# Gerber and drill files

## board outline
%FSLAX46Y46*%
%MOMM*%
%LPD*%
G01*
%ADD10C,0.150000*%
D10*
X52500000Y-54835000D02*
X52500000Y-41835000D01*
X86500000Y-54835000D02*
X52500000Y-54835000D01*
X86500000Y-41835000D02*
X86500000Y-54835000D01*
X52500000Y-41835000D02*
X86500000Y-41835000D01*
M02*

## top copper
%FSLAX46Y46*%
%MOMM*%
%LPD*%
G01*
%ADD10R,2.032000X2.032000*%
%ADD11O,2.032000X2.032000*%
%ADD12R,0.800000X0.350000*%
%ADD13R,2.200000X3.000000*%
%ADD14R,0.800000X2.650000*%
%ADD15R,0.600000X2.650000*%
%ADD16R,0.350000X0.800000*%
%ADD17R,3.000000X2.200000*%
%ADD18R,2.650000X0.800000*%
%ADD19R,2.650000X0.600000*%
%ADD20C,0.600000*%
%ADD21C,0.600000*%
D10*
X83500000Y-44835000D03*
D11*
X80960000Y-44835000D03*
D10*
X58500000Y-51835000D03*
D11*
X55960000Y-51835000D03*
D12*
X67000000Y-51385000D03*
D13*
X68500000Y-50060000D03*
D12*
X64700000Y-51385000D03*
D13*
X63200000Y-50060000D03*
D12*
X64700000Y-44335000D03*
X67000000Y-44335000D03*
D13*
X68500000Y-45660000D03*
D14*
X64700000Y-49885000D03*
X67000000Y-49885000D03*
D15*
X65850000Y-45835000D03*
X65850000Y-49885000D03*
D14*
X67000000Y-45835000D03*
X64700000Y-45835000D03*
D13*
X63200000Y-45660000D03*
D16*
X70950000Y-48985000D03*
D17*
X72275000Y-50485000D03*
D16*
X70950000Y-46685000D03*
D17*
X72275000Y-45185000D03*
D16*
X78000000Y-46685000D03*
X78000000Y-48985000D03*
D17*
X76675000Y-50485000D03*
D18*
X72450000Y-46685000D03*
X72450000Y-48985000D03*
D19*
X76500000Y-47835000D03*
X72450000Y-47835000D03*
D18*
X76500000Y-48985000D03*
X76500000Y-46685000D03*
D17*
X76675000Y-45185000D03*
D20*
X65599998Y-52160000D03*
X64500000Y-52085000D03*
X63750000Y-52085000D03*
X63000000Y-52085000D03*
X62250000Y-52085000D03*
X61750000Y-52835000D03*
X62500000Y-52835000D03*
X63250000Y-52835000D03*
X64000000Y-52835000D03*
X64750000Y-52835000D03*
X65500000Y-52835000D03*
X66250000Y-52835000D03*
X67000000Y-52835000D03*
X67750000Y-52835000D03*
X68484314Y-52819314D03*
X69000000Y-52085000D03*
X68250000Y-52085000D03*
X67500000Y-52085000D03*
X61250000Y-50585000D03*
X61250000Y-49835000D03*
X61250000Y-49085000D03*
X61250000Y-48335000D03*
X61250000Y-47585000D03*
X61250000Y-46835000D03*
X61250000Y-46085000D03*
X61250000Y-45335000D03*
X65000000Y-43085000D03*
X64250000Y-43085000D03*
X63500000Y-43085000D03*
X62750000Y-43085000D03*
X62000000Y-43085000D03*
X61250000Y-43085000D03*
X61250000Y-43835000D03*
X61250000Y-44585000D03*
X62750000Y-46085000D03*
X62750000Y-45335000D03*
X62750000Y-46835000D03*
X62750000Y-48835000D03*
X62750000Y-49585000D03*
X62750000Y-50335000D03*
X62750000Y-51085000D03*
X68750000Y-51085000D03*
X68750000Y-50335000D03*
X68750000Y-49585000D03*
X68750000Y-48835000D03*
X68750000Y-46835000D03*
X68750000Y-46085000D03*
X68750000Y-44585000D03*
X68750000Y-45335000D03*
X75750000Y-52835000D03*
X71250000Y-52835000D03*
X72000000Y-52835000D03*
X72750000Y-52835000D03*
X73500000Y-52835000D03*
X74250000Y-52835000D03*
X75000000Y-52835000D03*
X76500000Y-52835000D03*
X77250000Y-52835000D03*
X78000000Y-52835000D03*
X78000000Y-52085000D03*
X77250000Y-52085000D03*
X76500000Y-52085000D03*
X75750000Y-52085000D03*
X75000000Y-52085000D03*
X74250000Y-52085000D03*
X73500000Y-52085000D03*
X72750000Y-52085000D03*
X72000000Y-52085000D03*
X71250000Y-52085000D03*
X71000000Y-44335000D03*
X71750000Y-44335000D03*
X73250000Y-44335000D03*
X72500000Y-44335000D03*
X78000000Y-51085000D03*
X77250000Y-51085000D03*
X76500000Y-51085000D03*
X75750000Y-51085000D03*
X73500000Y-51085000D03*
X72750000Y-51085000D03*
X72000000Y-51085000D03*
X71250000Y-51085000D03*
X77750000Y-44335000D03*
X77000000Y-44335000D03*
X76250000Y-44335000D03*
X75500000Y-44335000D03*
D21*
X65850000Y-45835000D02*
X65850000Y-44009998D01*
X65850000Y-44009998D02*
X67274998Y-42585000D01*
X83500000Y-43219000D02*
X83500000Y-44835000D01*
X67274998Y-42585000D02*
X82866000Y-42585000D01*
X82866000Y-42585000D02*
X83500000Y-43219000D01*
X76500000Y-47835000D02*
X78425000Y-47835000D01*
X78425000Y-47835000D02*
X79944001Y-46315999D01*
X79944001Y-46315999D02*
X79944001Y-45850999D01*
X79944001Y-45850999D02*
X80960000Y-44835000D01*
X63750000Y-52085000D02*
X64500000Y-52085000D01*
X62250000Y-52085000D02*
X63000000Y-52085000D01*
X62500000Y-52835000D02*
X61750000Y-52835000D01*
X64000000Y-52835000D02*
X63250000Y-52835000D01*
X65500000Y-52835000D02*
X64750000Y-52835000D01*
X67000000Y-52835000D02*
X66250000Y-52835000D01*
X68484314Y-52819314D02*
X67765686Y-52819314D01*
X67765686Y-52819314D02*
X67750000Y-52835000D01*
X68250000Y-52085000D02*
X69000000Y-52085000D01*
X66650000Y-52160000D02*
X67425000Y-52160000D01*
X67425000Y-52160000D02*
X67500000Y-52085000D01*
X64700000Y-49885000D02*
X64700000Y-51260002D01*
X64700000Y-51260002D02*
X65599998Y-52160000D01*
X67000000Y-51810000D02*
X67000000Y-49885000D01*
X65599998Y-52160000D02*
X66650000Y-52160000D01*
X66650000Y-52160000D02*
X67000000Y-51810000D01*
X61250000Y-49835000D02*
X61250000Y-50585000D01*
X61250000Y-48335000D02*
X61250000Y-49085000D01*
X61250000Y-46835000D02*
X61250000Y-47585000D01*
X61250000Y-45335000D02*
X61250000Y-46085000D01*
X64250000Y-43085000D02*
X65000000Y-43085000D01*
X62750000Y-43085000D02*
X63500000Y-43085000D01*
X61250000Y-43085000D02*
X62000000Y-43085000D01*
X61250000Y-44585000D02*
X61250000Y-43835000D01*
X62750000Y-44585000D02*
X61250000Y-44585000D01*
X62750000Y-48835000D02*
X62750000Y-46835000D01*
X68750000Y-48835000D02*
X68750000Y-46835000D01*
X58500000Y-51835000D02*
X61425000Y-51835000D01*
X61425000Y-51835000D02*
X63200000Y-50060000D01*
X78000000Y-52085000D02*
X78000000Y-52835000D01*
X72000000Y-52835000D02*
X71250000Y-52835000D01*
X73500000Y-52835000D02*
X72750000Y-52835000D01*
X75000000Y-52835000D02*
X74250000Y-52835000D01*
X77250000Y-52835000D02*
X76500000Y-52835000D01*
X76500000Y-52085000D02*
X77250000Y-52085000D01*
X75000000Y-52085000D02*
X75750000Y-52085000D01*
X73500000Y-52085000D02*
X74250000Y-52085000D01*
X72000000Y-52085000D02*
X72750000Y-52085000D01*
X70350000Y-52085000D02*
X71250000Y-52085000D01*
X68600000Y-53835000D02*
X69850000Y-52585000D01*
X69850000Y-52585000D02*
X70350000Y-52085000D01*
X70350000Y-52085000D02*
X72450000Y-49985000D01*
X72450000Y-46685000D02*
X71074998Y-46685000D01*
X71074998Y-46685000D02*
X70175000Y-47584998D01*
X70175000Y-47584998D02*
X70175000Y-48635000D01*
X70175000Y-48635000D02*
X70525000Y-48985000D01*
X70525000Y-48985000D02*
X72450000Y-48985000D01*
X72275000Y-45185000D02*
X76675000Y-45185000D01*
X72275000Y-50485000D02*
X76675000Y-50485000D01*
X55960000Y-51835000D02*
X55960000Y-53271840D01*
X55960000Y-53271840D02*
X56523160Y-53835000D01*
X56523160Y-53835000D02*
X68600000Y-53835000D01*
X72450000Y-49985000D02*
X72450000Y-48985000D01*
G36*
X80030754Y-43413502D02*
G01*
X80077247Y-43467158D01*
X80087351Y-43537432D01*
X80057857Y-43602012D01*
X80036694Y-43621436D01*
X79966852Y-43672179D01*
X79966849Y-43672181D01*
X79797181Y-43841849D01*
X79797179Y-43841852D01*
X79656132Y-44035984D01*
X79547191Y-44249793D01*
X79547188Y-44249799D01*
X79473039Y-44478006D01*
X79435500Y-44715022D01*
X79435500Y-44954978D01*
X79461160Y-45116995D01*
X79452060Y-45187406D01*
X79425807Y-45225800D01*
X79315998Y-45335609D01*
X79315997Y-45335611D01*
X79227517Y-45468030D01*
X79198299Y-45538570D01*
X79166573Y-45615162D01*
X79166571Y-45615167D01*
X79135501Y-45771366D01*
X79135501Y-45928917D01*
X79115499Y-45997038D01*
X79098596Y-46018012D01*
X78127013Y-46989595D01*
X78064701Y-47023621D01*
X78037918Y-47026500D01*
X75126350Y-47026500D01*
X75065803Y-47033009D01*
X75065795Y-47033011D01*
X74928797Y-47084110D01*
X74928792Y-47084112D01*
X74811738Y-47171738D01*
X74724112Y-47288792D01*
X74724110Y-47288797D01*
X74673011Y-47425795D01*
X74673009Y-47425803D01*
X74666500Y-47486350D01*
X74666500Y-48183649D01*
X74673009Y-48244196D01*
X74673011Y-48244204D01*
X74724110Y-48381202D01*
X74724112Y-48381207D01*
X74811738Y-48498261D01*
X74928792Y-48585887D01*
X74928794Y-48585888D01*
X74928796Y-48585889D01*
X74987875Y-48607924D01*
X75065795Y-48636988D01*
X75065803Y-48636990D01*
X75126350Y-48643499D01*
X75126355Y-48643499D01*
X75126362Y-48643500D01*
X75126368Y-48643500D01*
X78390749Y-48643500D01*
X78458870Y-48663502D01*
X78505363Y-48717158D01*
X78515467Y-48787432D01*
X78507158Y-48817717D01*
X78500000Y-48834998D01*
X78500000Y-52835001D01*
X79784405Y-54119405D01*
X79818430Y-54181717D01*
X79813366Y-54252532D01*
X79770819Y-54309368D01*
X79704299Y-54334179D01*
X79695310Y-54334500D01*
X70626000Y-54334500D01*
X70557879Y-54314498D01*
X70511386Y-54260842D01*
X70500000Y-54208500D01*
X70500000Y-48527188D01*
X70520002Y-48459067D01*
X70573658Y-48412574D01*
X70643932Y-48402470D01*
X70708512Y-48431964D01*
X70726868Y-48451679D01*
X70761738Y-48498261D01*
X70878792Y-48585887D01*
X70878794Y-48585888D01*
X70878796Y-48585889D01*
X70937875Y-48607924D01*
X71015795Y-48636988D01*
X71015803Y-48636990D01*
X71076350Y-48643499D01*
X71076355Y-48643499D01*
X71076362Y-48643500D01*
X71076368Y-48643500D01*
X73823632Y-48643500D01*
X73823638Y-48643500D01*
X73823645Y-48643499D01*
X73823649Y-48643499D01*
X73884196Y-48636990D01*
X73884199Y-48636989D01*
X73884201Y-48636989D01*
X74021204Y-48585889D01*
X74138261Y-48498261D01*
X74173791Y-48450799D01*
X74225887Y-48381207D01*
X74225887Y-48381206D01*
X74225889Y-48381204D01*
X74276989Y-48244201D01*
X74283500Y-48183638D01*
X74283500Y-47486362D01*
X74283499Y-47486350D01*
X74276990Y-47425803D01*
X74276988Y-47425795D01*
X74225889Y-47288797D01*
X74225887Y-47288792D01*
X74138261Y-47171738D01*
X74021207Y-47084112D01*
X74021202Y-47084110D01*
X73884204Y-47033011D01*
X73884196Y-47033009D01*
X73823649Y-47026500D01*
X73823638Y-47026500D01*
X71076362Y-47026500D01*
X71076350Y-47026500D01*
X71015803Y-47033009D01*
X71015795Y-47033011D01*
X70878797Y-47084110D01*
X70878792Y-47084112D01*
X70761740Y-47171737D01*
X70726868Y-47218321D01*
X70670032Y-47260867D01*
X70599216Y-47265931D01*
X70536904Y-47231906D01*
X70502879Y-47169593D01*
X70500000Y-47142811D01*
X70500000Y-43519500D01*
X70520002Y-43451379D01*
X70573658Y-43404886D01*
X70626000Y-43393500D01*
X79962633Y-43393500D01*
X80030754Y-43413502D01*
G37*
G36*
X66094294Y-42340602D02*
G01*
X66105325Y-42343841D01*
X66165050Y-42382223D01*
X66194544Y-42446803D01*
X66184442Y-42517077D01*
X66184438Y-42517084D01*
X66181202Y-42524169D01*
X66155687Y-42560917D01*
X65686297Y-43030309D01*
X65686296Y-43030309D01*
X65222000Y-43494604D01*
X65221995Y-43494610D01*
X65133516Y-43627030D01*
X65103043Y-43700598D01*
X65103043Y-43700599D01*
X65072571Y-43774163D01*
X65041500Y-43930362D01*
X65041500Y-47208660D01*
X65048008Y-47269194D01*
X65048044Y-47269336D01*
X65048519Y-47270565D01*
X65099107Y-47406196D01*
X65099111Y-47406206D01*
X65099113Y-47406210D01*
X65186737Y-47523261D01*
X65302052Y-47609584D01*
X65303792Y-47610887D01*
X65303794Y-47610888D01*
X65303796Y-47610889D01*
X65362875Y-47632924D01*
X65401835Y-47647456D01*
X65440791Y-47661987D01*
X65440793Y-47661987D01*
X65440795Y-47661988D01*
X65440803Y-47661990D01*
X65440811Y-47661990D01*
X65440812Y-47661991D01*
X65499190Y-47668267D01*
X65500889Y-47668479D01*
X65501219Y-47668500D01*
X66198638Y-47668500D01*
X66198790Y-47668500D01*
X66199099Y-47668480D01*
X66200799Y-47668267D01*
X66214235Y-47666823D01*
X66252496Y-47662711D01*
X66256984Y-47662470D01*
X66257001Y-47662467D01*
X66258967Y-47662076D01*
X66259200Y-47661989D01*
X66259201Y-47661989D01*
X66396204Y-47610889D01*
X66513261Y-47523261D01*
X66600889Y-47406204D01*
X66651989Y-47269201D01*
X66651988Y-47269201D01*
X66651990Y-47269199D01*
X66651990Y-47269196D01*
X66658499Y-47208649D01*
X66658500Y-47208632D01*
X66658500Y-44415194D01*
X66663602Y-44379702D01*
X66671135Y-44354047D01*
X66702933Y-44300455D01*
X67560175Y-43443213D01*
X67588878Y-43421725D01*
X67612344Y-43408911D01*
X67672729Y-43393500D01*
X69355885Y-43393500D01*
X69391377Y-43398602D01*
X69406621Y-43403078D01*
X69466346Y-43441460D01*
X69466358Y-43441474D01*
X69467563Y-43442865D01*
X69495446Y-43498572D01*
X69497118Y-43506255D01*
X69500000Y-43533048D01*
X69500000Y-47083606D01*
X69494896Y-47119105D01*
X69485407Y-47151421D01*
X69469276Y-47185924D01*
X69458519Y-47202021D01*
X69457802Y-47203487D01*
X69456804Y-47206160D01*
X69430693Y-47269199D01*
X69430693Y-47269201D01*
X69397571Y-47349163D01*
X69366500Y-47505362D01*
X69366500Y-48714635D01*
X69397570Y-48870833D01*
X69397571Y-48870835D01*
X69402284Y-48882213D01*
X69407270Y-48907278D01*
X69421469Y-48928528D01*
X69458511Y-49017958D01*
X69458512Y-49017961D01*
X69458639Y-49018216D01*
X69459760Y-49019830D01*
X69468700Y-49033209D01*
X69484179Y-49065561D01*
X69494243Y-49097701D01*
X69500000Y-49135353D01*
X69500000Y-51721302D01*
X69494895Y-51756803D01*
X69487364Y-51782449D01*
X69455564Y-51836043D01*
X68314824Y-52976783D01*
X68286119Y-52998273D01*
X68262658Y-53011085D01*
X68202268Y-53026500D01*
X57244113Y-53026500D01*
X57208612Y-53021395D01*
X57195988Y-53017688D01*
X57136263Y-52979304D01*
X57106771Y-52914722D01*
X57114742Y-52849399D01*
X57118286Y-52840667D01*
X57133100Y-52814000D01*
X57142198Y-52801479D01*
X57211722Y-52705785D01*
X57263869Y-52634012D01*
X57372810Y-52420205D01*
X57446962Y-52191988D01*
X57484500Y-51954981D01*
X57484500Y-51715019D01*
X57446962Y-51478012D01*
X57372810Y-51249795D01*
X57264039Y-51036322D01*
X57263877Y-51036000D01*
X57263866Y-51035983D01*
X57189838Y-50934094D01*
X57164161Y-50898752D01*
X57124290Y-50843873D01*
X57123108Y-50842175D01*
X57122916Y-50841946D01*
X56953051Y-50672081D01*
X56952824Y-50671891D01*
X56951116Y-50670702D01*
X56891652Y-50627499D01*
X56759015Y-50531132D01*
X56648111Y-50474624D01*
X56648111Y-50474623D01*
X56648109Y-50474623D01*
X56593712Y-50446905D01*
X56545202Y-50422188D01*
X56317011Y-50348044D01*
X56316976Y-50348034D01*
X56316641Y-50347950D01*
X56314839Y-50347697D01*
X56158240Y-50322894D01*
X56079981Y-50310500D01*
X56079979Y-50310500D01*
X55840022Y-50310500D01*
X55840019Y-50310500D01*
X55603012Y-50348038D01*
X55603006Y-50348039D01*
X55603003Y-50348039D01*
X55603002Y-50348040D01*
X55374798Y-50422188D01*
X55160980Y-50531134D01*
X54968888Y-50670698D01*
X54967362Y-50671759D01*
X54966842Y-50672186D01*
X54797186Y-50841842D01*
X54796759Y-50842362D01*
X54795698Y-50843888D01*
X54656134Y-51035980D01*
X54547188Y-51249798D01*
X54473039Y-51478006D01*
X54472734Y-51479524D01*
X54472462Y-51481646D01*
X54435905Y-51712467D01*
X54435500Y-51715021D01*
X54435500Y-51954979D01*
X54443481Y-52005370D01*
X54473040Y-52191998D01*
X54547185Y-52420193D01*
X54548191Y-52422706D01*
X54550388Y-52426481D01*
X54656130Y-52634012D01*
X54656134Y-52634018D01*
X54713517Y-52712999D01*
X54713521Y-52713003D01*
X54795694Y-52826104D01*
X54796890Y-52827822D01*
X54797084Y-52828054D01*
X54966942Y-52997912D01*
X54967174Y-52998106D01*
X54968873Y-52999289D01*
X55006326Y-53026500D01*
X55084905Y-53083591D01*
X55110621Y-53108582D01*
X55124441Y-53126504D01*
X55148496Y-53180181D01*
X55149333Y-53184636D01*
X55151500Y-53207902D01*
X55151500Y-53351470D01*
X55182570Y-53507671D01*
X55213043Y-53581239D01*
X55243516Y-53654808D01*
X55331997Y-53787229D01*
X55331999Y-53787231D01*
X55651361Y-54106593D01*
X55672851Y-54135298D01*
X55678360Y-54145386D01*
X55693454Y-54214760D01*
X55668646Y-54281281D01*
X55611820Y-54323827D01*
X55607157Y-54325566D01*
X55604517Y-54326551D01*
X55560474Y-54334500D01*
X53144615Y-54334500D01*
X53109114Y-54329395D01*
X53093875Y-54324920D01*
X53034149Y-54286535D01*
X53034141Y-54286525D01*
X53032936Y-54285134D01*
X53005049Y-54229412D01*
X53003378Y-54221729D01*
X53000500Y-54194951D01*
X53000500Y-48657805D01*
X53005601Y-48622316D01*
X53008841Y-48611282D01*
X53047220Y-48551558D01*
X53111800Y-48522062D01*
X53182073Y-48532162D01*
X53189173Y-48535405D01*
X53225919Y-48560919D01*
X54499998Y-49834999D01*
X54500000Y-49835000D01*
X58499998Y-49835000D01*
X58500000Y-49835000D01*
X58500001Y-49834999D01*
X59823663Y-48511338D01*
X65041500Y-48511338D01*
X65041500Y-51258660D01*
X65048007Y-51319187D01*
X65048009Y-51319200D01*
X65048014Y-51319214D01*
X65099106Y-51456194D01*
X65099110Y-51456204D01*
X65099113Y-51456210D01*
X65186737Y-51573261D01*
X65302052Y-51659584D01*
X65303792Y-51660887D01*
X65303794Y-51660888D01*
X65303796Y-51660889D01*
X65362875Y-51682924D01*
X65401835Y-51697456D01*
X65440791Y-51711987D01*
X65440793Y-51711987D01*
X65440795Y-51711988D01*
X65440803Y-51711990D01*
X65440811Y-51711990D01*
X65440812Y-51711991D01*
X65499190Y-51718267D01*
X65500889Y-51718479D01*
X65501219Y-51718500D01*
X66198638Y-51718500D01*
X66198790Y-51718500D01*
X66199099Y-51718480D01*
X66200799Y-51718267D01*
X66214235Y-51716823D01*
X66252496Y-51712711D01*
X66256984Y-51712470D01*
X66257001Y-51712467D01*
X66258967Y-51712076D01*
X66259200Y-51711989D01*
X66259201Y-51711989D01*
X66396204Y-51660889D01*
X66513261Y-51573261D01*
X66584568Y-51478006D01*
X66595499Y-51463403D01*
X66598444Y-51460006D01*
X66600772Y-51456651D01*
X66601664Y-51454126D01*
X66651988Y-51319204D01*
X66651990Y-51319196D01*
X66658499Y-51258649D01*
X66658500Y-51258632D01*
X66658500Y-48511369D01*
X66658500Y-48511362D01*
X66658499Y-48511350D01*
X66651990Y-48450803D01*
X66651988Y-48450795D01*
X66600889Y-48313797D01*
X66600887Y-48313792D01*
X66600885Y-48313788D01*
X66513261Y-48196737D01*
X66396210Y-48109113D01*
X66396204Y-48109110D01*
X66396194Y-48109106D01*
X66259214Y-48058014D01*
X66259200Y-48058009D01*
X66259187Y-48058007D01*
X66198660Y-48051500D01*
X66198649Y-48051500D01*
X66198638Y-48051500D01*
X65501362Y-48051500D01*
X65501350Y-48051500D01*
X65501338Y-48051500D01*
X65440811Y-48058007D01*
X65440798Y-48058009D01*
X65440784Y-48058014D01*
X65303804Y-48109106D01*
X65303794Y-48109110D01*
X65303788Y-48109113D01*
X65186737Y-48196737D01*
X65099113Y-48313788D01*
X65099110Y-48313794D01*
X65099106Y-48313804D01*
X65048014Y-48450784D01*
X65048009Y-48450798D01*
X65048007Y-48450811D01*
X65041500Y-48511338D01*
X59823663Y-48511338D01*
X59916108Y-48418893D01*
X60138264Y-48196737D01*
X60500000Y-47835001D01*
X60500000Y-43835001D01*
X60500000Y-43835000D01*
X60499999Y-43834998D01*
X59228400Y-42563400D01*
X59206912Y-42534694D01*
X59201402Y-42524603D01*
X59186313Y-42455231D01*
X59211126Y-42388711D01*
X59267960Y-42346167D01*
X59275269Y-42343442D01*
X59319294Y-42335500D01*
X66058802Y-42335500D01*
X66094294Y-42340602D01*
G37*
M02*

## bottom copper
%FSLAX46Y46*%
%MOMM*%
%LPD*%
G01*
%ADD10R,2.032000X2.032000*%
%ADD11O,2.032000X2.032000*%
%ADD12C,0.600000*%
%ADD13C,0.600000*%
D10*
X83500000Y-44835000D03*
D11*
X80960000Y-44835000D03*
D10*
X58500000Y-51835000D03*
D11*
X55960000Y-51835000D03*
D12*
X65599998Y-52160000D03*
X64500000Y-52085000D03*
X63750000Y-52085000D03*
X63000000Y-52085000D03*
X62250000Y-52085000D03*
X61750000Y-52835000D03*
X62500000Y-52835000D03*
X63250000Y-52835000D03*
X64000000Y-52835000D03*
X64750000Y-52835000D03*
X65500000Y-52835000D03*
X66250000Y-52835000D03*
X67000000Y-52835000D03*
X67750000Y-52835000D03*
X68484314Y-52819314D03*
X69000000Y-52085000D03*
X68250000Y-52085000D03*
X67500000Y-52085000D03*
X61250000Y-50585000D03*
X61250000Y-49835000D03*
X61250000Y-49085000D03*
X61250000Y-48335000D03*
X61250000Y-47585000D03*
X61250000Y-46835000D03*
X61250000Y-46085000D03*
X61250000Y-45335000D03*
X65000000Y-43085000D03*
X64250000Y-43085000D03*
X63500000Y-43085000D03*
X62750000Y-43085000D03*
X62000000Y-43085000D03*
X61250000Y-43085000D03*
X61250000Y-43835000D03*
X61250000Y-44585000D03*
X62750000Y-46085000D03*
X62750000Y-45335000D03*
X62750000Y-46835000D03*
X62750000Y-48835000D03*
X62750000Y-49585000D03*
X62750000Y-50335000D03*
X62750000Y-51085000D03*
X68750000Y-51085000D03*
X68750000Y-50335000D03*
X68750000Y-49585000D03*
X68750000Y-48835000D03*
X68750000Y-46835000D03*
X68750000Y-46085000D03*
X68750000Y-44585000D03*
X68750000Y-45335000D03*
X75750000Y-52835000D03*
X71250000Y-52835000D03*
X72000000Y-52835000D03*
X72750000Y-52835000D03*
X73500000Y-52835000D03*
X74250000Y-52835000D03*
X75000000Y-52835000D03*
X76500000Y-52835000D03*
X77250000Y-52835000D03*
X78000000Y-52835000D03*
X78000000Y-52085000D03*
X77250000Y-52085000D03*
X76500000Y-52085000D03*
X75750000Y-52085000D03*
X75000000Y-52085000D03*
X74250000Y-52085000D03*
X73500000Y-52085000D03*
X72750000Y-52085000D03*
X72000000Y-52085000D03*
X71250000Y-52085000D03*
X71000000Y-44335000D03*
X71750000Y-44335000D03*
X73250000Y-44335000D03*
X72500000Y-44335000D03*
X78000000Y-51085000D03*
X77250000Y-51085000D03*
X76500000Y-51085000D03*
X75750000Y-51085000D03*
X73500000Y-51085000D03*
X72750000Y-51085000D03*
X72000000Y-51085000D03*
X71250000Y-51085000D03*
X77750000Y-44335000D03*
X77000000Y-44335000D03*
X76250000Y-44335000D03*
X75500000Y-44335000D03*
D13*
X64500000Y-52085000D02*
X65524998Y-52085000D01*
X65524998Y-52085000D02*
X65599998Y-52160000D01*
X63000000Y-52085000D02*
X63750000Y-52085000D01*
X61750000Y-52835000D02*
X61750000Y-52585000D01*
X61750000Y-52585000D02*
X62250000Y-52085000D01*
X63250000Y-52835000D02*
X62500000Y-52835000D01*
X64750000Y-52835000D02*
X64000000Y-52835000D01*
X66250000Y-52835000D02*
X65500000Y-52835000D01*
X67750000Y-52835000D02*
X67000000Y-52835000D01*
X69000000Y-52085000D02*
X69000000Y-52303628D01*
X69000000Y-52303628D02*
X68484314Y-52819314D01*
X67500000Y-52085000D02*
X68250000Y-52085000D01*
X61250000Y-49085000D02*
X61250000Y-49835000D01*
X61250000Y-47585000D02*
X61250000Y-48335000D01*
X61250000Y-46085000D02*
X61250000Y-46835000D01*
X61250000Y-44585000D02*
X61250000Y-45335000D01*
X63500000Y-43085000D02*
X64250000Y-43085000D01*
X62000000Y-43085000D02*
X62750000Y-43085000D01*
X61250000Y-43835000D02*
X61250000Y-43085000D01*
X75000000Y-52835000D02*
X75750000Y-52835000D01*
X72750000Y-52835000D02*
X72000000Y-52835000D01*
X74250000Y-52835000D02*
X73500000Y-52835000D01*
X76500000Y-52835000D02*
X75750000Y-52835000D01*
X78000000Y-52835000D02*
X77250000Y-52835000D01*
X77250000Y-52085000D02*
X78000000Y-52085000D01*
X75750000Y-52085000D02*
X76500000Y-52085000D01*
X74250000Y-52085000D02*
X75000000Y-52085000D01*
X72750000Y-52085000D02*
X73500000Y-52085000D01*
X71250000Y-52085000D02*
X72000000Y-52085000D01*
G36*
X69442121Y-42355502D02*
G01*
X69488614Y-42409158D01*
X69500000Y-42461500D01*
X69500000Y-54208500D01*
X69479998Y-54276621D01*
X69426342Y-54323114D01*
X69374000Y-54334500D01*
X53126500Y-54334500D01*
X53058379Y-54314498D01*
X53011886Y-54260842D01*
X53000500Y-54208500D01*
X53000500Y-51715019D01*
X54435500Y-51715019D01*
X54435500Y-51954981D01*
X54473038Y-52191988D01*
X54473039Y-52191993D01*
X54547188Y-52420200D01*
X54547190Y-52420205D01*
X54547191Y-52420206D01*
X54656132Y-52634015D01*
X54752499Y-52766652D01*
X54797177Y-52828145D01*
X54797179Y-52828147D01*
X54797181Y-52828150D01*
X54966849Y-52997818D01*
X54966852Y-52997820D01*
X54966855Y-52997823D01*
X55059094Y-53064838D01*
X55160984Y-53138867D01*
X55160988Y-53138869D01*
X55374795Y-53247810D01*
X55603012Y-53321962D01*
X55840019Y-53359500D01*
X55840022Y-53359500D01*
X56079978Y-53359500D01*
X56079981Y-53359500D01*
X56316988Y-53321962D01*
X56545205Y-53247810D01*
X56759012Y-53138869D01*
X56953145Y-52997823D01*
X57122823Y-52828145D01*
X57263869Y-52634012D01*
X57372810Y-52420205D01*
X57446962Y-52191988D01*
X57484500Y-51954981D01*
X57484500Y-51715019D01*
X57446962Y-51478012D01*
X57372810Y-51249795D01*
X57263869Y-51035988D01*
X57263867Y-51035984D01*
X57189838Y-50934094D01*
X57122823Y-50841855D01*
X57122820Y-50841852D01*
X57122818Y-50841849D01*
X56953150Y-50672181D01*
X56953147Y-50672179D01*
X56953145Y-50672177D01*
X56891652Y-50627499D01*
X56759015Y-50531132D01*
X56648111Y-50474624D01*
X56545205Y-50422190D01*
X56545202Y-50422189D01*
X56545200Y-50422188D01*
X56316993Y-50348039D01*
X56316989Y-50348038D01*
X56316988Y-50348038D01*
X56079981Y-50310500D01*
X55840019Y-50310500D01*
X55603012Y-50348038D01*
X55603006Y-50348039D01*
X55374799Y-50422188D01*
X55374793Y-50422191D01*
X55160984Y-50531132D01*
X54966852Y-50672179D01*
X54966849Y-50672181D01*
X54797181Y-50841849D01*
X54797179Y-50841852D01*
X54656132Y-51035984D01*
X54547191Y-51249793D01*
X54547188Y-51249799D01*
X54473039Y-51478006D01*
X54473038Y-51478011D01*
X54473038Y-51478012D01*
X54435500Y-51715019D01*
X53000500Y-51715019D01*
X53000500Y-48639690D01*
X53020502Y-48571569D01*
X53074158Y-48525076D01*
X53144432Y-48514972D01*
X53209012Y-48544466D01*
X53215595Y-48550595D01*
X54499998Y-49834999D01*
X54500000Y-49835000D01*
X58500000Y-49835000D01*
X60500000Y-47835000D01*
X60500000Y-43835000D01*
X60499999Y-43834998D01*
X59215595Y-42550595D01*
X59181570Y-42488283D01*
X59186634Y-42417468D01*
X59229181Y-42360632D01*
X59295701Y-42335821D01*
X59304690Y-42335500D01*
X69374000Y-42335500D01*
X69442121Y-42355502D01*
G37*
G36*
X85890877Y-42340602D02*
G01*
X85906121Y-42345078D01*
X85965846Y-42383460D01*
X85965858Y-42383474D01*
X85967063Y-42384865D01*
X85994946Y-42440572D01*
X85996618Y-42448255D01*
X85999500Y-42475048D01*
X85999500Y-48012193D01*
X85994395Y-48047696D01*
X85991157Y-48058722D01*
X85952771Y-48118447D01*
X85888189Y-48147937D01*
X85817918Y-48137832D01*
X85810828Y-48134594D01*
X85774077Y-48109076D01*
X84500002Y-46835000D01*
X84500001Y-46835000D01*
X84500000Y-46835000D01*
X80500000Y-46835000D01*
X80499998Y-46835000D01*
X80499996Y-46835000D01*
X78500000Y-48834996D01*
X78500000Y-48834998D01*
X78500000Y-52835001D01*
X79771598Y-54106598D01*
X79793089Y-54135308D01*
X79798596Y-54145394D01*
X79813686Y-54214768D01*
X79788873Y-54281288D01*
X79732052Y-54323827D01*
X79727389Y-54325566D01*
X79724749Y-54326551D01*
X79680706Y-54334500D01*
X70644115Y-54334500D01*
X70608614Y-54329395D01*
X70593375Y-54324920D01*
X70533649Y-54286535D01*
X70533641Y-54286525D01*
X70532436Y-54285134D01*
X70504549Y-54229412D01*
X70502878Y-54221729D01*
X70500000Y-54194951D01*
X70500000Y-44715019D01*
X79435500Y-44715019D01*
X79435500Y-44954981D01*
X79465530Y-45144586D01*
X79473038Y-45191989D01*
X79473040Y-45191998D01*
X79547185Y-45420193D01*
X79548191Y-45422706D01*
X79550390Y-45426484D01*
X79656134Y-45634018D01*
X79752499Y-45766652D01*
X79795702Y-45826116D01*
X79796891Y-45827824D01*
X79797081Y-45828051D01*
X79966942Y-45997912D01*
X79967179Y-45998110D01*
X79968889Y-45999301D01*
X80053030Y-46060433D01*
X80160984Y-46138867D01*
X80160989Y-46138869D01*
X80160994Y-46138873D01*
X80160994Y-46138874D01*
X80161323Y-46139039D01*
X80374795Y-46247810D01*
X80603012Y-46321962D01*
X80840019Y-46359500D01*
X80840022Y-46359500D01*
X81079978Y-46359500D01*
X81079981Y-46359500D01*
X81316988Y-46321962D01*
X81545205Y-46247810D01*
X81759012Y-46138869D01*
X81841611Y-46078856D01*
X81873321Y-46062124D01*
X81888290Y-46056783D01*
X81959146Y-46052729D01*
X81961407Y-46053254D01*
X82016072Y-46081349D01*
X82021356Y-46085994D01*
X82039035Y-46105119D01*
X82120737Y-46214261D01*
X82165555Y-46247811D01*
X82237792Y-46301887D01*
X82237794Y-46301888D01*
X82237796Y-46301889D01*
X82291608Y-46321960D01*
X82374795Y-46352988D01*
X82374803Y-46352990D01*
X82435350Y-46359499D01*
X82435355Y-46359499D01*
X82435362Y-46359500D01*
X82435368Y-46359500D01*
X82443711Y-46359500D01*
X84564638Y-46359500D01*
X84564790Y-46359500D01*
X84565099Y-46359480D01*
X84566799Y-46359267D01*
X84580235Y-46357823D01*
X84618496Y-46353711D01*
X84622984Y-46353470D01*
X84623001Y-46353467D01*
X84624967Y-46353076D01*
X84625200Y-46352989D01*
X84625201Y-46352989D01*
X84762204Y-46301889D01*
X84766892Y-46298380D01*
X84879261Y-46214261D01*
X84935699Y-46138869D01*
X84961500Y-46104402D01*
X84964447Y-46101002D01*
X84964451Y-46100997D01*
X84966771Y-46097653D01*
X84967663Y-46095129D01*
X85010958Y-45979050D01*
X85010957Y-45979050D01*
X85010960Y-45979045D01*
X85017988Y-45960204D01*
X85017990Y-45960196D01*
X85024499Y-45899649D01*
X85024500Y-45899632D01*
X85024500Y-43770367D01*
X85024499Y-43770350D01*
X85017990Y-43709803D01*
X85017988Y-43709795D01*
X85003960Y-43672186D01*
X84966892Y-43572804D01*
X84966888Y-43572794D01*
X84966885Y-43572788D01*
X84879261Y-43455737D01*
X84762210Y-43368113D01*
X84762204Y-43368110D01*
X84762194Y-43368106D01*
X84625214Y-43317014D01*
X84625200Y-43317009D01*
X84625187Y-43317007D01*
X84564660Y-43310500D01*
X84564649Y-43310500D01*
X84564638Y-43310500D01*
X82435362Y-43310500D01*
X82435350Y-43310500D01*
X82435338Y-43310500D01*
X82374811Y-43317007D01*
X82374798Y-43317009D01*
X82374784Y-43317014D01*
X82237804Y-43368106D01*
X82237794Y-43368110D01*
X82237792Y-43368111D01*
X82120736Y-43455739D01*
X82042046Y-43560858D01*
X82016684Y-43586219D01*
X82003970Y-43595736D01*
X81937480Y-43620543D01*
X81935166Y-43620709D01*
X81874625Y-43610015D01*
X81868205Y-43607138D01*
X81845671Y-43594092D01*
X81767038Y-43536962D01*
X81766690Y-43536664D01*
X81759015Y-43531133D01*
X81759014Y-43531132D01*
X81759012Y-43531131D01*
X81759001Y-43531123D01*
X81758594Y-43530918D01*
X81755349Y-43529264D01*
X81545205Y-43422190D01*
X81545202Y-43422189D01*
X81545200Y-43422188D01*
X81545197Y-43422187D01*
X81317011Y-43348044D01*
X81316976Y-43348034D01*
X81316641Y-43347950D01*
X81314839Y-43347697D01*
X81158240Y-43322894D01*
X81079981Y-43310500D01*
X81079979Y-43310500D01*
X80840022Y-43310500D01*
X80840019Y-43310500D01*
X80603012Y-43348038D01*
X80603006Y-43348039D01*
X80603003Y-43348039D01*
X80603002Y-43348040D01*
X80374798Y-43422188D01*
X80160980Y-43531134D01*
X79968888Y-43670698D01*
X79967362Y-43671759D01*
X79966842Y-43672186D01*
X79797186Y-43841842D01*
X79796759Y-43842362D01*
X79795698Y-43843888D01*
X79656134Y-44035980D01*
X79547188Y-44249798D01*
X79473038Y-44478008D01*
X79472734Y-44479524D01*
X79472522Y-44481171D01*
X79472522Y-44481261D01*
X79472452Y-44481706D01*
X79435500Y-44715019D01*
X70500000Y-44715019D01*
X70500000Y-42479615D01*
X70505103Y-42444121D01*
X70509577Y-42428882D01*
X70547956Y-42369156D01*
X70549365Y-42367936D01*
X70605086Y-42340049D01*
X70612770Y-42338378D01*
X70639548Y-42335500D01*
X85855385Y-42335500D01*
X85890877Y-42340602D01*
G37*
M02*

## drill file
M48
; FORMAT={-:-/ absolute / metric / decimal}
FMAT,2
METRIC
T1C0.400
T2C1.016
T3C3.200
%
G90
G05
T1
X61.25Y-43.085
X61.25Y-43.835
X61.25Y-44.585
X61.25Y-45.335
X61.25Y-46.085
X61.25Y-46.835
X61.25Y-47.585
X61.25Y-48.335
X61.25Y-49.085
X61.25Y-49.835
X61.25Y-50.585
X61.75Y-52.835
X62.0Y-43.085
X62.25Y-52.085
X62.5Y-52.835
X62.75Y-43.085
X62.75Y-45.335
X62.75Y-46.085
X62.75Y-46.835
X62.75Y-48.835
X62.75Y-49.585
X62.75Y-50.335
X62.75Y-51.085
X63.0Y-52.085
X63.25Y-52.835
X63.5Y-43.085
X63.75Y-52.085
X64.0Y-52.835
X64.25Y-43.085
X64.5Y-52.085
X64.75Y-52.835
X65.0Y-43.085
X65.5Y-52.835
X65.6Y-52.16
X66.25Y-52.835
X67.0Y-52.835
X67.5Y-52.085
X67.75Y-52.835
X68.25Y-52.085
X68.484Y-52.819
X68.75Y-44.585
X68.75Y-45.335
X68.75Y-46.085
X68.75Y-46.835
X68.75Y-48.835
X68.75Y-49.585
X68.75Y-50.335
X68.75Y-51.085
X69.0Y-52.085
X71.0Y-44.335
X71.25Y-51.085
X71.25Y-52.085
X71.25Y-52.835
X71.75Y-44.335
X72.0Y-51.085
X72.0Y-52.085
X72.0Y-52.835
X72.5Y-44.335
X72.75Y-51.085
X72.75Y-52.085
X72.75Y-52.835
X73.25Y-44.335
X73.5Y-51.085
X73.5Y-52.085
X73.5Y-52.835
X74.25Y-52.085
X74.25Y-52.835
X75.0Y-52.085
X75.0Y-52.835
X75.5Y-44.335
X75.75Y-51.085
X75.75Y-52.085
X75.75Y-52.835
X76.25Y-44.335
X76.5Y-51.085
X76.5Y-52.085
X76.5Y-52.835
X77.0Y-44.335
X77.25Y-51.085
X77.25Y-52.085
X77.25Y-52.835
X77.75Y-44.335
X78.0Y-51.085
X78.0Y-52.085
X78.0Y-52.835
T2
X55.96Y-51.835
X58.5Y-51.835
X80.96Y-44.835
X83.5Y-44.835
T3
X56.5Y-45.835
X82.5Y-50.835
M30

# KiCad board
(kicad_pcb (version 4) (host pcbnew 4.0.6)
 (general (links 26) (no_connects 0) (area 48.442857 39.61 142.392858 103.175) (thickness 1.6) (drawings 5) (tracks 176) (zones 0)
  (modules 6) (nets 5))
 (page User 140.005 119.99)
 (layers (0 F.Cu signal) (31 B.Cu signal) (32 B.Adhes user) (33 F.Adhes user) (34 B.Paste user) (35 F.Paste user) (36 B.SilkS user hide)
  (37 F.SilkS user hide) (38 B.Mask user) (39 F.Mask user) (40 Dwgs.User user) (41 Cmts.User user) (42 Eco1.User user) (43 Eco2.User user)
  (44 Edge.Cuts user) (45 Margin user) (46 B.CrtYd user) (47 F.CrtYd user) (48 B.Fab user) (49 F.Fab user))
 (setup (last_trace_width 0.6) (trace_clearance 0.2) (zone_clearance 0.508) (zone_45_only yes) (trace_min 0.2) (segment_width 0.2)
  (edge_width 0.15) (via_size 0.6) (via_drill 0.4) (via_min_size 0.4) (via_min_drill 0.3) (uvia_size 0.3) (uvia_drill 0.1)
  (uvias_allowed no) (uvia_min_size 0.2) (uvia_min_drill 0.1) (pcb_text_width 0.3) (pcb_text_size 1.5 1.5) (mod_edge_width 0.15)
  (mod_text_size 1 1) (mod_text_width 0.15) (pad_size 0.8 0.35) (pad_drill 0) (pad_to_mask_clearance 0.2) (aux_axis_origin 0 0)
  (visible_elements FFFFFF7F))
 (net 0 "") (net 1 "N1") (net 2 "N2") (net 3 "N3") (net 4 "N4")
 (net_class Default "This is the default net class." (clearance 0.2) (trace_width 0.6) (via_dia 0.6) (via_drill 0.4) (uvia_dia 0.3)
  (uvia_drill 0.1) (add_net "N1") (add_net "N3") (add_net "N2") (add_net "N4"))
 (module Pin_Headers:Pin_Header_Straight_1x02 (layer F.Cu) (at 83.5 44.835 270)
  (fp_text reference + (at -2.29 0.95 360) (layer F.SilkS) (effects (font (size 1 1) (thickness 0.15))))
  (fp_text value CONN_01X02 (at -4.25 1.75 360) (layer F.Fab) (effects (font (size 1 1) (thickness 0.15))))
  (pad 1 thru_hole rect (at 0 0 270) (size 2.032 2.032) (drill 1.016) (layers *.Cu *.Mask) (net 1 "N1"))
  (pad 2 thru_hole oval (at 0 2.54 270) (size 2.032 2.032) (drill 1.016) (layers *.Cu *.Mask) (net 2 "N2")))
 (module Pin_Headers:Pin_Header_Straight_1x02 (layer F.Cu) (at 58.5 51.835 270)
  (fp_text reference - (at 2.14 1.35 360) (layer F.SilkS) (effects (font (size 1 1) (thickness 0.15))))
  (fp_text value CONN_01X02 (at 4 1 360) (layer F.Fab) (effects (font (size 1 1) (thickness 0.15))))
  (pad 1 thru_hole rect (at 0 0 270) (size 2.032 2.032) (drill 1.016) (layers *.Cu *.Mask) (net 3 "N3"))
  (pad 2 thru_hole oval (at 0 2.54 270) (size 2.032 2.032) (drill 1.016) (layers *.Cu *.Mask) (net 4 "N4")))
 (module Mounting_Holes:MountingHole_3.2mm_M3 (layer F.Cu) (at 82.5 50.835)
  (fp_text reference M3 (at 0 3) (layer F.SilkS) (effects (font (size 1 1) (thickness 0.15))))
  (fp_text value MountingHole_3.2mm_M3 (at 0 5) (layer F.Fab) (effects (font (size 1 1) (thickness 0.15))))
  (pad 1 np_thru_hole circle (at 0 0) (size 3.2 3.2) (drill 3.2) (layers *.Cu *.Mask)))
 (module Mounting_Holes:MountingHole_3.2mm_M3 (layer F.Cu) (at 56.5 45.835)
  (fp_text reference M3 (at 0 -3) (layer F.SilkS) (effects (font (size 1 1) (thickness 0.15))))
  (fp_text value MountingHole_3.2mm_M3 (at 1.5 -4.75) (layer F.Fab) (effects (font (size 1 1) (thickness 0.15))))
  (pad 1 np_thru_hole circle (at 0 0) (size 3.2 3.2) (drill 3.2) (layers *.Cu *.Mask)))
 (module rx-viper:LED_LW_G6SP (layer F.Cu) (at 64.7 45.835)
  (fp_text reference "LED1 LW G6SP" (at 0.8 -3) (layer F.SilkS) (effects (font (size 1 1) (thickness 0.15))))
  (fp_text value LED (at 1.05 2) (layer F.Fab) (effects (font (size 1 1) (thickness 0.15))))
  (pad ~ smd rect (at 2.3 5.55) (size 0.8 0.35) (layers F.Cu) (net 3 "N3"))
  (pad ~ smd rect (at 3.8 4.225) (size 2.2 3) (layers F.Cu) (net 3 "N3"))
  (pad ~ smd rect (at 0 5.55) (size 0.8 0.35) (layers F.Cu) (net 3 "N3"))
  (pad ~ smd rect (at -1.5 4.225) (size 2.2 3) (layers F.Cu) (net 3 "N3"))
  (pad ~ smd rect (at 0 -1.5) (size 0.8 0.35) (layers F.Cu) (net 3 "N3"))
  (pad ~ smd rect (at 2.3 -1.5) (size 0.8 0.35) (layers F.Cu) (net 3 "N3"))
  (pad ~ smd rect (at 3.8 -0.175) (size 2.2 3) (layers F.Cu) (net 3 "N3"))
  (pad 2 smd rect (at 0 4.05) (size 0.8 2.65) (layers F.Cu F.Mask) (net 3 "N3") (solder_mask_margin 0.1))
  (pad 2 smd rect (at 2.3 4.05) (size 0.8 2.65) (layers F.Cu F.Mask) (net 3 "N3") (solder_mask_margin 0.1))
  (pad 1 smd rect (at 1.15 0) (size 0.6 2.65) (layers F.Cu F.Mask) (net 1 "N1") (solder_mask_margin 0.1))
  (pad ~ smd rect (at 1.15 4.05) (size 0.6 2.65) (layers F.Cu F.Mask) (solder_mask_margin 0.1))
  (pad 2 smd rect (at 2.3 0) (size 0.8 2.65) (layers F.Cu F.Mask) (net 3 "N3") (solder_mask_margin 0.1))
  (pad 2 smd rect (at 0 0) (size 0.8 2.65) (layers F.Cu F.Mask) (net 3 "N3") (solder_mask_margin 0.1))
  (pad ~ smd rect (at -1.5 -0.175) (size 2.2 3) (layers F.Cu) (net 3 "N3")))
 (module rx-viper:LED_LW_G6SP (layer F.Cu) (at 76.5 46.685 270)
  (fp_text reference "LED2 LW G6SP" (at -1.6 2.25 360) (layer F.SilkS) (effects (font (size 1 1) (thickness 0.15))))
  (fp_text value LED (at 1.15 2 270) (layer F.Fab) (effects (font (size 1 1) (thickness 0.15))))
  (pad ~ smd rect (at 2.3 5.55 270) (size 0.8 0.35) (layers F.Cu) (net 4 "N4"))
  (pad ~ smd rect (at 3.8 4.225 270) (size 2.2 3) (layers F.Cu) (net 4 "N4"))
  (pad ~ smd rect (at 0 5.55 270) (size 0.8 0.35) (layers F.Cu) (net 4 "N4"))
  (pad ~ smd rect (at -1.5 4.225 270) (size 2.2 3) (layers F.Cu) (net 4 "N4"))
  (pad ~ smd rect (at 0 -1.5 270) (size 0.8 0.35) (layers F.Cu) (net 4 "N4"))
  (pad ~ smd rect (at 2.3 -1.5 270) (size 0.8 0.35) (layers F.Cu) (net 4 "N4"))
  (pad ~ smd rect (at 3.8 -0.175 270) (size 2.2 3) (layers F.Cu) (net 4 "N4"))
  (pad 2 smd rect (at 0 4.05 270) (size 0.8 2.65) (layers F.Cu F.Mask) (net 4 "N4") (solder_mask_margin 0.1))
  (pad 2 smd rect (at 2.3 4.05 270) (size 0.8 2.65) (layers F.Cu F.Mask) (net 4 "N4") (solder_mask_margin 0.1))
  (pad 1 smd rect (at 1.15 0 270) (size 0.6 2.65) (layers F.Cu F.Mask) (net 2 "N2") (solder_mask_margin 0.1))
  (pad ~ smd rect (at 1.15 4.05 270) (size 0.6 2.65) (layers F.Cu F.Mask) (solder_mask_margin 0.1))
  (pad 2 smd rect (at 2.3 0 270) (size 0.8 2.65) (layers F.Cu F.Mask) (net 4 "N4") (solder_mask_margin 0.1))
  (pad 2 smd rect (at 0 0 270) (size 0.8 2.65) (layers F.Cu F.Mask) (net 4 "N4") (solder_mask_margin 0.1))
  (pad ~ smd rect (at -1.5 -0.175 270) (size 2.2 3) (layers F.Cu) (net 4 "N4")))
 (gr_line (start 52.5 54.835) (end 52.5 41.835) (layer Edge.Cuts) (width 0.15))
 (gr_line (start 86.5 54.835) (end 52.5 54.835) (layer Edge.Cuts) (width 0.15))
 (gr_line (start 86.5 41.835) (end 86.5 54.835) (layer Edge.Cuts) (width 0.15))
 (gr_line (start 52.5 41.835) (end 86.5 41.835) (layer Edge.Cuts) (width 0.15))
 (segment (start 65.85 45.835) (end 65.85 44.009998) (width 0.6) (layer F.Cu) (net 1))
 (segment (start 65.85 44.009998) (end 67.274998 42.585) (width 0.6) (layer F.Cu) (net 1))
 (segment (start 83.5 43.219) (end 83.5 44.835) (width 0.6) (layer F.Cu) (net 1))
 (segment (start 67.274998 42.585) (end 82.866 42.585) (width 0.6) (layer F.Cu) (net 1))
 (segment (start 82.866 42.585) (end 83.5 43.219) (width 0.6) (layer F.Cu) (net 1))
 (segment (start 76.5 47.835) (end 78.425 47.835) (width 0.6) (layer F.Cu) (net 2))
 (segment (start 78.425 47.835) (end 79.944001 46.315999) (width 0.6) (layer F.Cu) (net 2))
 (segment (start 79.944001 46.315999) (end 79.944001 45.850999) (width 0.6) (layer F.Cu) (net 2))
 (segment (start 79.944001 45.850999) (end 80.96 44.835) (width 0.6) (layer F.Cu) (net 2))
 (segment (start 64.5 52.085) (end 65.524998 52.085) (width 0.6) (layer B.Cu) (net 3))
 (segment (start 65.524998 52.085) (end 65.599998 52.16) (width 0.6) (layer B.Cu) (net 3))
 (via (at 65.599998 52.16) (size 0.6) (drill 0.4) (layers F.Cu B.Cu) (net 3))
 (segment (start 63.75 52.085) (end 64.5 52.085) (width 0.6) (layer F.Cu) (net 3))
 (via (at 64.5 52.085) (size 0.6) (drill 0.4) (layers F.Cu B.Cu) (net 3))
 (segment (start 63 52.085) (end 63.75 52.085) (width 0.6) (layer B.Cu) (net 3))
 (via (at 63.75 52.085) (size 0.6) (drill 0.4) (layers F.Cu B.Cu) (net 3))
 (segment (start 62.25 52.085) (end 63 52.085) (width 0.6) (layer F.Cu) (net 3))
 (via (at 63 52.085) (size 0.6) (drill 0.4) (layers F.Cu B.Cu) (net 3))
 (segment (start 61.75 52.835) (end 61.75 52.585) (width 0.6) (layer B.Cu) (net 3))
 (via (at 62.25 52.085) (size 0.6) (drill 0.4) (layers F.Cu B.Cu) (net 3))
 (segment (start 61.75 52.585) (end 62.25 52.085) (width 0.6) (layer B.Cu) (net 3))
 (segment (start 62.5 52.835) (end 61.75 52.835) (width 0.6) (layer F.Cu) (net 3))
 (via (at 61.75 52.835) (size 0.6) (drill 0.4) (layers F.Cu B.Cu) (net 3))
 (segment (start 63.25 52.835) (end 62.5 52.835) (width 0.6) (layer B.Cu) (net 3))
 (via (at 62.5 52.835) (size 0.6) (drill 0.4) (layers F.Cu B.Cu) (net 3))
 (segment (start 64 52.835) (end 63.25 52.835) (width 0.6) (layer F.Cu) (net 3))
 (via (at 63.25 52.835) (size 0.6) (drill 0.4) (layers F.Cu B.Cu) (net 3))
 (segment (start 64.75 52.835) (end 64 52.835) (width 0.6) (layer B.Cu) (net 3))
 (via (at 64 52.835) (size 0.6) (drill 0.4) (layers F.Cu B.Cu) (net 3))
 (segment (start 65.5 52.835) (end 64.75 52.835) (width 0.6) (layer F.Cu) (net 3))
 (via (at 64.75 52.835) (size 0.6) (drill 0.4) (layers F.Cu B.Cu) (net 3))
 (segment (start 66.25 52.835) (end 65.5 52.835) (width 0.6) (layer B.Cu) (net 3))
 (via (at 65.5 52.835) (size 0.6) (drill 0.4) (layers F.Cu B.Cu) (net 3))
 (segment (start 67 52.835) (end 66.25 52.835) (width 0.6) (layer F.Cu) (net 3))
 (via (at 66.25 52.835) (size 0.6) (drill 0.4) (layers F.Cu B.Cu) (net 3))
 (segment (start 67.75 52.835) (end 67 52.835) (width 0.6) (layer B.Cu) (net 3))
 (via (at 67 52.835) (size 0.6) (drill 0.4) (layers F.Cu B.Cu) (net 3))
 (segment (start 68.484314 52.819314) (end 67.765686 52.819314) (width 0.6) (layer F.Cu) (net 3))
 (segment (start 67.765686 52.819314) (end 67.75 52.835) (width 0.6) (layer F.Cu) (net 3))
 (via (at 67.75 52.835) (size 0.6) (drill 0.4) (layers F.Cu B.Cu) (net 3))
 (segment (start 69 52.085) (end 69 52.303628) (width 0.6) (layer B.Cu) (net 3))
 (segment (start 69 52.303628) (end 68.484314 52.819314) (width 0.6) (layer B.Cu) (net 3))
 (via (at 68.484314 52.819314) (size 0.6) (drill 0.4) (layers F.Cu B.Cu) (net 3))
 (segment (start 68.25 52.085) (end 69 52.085) (width 0.6) (layer F.Cu) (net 3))
 (via (at 69 52.085) (size 0.6) (drill 0.4) (layers F.Cu B.Cu) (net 3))
 (segment (start 67.5 52.085) (end 68.25 52.085) (width 0.6) (layer B.Cu) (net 3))
 (via (at 68.25 52.085) (size 0.6) (drill 0.4) (layers F.Cu B.Cu) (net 3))
 (segment (start 66.65 52.16) (end 67.425 52.16) (width 0.6) (layer F.Cu) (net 3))
 (segment (start 67.425 52.16) (end 67.5 52.085) (width 0.6) (layer F.Cu) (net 3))
 (via (at 67.5 52.085) (size 0.6) (drill 0.4) (layers F.Cu B.Cu) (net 3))
 (segment (start 64.7 49.885) (end 64.7 51.260002) (width 0.6) (layer F.Cu) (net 3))
 (segment (start 64.7 51.260002) (end 65.599998 52.16) (width 0.6) (layer F.Cu) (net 3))
 (segment (start 67 51.81) (end 67 49.885) (width 0.6) (layer F.Cu) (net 3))
 (segment (start 65.599998 52.16) (end 66.65 52.16) (width 0.6) (layer F.Cu) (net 3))
 (segment (start 66.65 52.16) (end 67 51.81) (width 0.6) (layer F.Cu) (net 3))
 (segment (start 61.25 49.835) (end 61.25 50.585) (width 0.6) (layer F.Cu) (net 3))
 (via (at 61.25 50.585) (size 0.6) (drill 0.4) (layers F.Cu B.Cu) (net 3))
 (segment (start 61.25 49.085) (end 61.25 49.835) (width 0.6) (layer B.Cu) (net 3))
 (via (at 61.25 49.835) (size 0.6) (drill 0.4) (layers F.Cu B.Cu) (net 3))
 (segment (start 61.25 48.335) (end 61.25 49.085) (width 0.6) (layer F.Cu) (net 3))
 (via (at 61.25 49.085) (size 0.6) (drill 0.4) (layers F.Cu B.Cu) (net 3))
 (segment (start 61.25 47.585) (end 61.25 48.335) (width 0.6) (layer B.Cu) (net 3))
 (via (at 61.25 48.335) (size 0.6) (drill 0.4) (layers F.Cu B.Cu) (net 3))
 (segment (start 61.25 46.835) (end 61.25 47.585) (width 0.6) (layer F.Cu) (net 3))
 (via (at 61.25 47.585) (size 0.6) (drill 0.4) (layers F.Cu B.Cu) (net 3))
 (segment (start 61.25 46.085) (end 61.25 46.835) (width 0.6) (layer B.Cu) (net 3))
 (via (at 61.25 46.835) (size 0.6) (drill 0.4) (layers F.Cu B.Cu) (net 3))
 (segment (start 61.25 45.335) (end 61.25 46.085) (width 0.6) (layer F.Cu) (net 3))
 (via (at 61.25 46.085) (size 0.6) (drill 0.4) (layers F.Cu B.Cu) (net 3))
 (segment (start 61.25 44.585) (end 61.25 45.335) (width 0.6) (layer B.Cu) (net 3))
 (via (at 61.25 45.335) (size 0.6) (drill 0.4) (layers F.Cu B.Cu) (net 3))
 (segment (start 64.25 43.085) (end 65 43.085) (width 0.6) (layer F.Cu) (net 3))
 (via (at 65 43.085) (size 0.6) (drill 0.4) (layers F.Cu B.Cu) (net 3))
 (segment (start 63.5 43.085) (end 64.25 43.085) (width 0.6) (layer B.Cu) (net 3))
 (via (at 64.25 43.085) (size 0.6) (drill 0.4) (layers F.Cu B.Cu) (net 3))
 (segment (start 62.75 43.085) (end 63.5 43.085) (width 0.6) (layer F.Cu) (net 3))
 (via (at 63.5 43.085) (size 0.6) (drill 0.4) (layers F.Cu B.Cu) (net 3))
 (segment (start 62 43.085) (end 62.75 43.085) (width 0.6) (layer B.Cu) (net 3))
 (via (at 62.75 43.085) (size 0.6) (drill 0.4) (layers F.Cu B.Cu) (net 3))
 (segment (start 61.25 43.085) (end 62 43.085) (width 0.6) (layer F.Cu) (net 3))
 (via (at 62 43.085) (size 0.6) (drill 0.4) (layers F.Cu B.Cu) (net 3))
 (segment (start 61.25 43.835) (end 61.25 43.085) (width 0.6) (layer B.Cu) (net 3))
 (via (at 61.25 43.085) (size 0.6) (drill 0.4) (layers F.Cu B.Cu) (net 3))
 (segment (start 61.25 44.585) (end 61.25 43.835) (width 0.6) (layer F.Cu) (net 3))
 (via (at 61.25 43.835) (size 0.6) (drill 0.4) (layers F.Cu B.Cu) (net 3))
 (segment (start 62.75 44.585) (end 61.25 44.585) (width 0.6) (layer F.Cu) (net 3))
 (via (at 61.25 44.585) (size 0.6) (drill 0.4) (layers F.Cu B.Cu) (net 3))
 (segment (start 62.75 48.835) (end 62.75 46.835) (width 0.6) (layer F.Cu) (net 3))
 (segment (start 68.75 48.835) (end 68.75 46.835) (width 0.6) (layer F.Cu) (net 3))
 (segment (start 58.5 51.835) (end 61.425 51.835) (width 0.6) (layer F.Cu) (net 3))
 (segment (start 61.425 51.835) (end 63.2 50.06) (width 0.6) (layer F.Cu) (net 3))
 (via (at 62.75 46.085) (size 0.6) (drill 0.4) (layers F.Cu B.Cu) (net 3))
 (via (at 62.75 45.335) (size 0.6) (drill 0.4) (layers F.Cu B.Cu) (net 3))
 (via (at 62.75 46.835) (size 0.6) (drill 0.4) (layers F.Cu B.Cu) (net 3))
 (via (at 62.75 48.835) (size 0.6) (drill 0.4) (layers F.Cu B.Cu) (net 3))
 (via (at 62.75 49.585) (size 0.6) (drill 0.4) (layers F.Cu B.Cu) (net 3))
 (via (at 62.75 50.335) (size 0.6) (drill 0.4) (layers F.Cu B.Cu) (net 3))
 (via (at 62.75 51.085) (size 0.6) (drill 0.4) (layers F.Cu B.Cu) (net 3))
 (via (at 68.75 51.085) (size 0.6) (drill 0.4) (layers F.Cu B.Cu) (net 3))
 (via (at 68.75 50.335) (size 0.6) (drill 0.4) (layers F.Cu B.Cu) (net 3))
 (via (at 68.75 49.585) (size 0.6) (drill 0.4) (layers F.Cu B.Cu) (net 3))
 (via (at 68.75 48.835) (size 0.6) (drill 0.4) (layers F.Cu B.Cu) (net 3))
 (via (at 68.75 46.835) (size 0.6) (drill 0.4) (layers F.Cu B.Cu) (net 3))
 (via (at 68.75 46.085) (size 0.6) (drill 0.4) (layers F.Cu B.Cu) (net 3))
 (via (at 68.75 44.585) (size 0.6) (drill 0.4) (layers F.Cu B.Cu) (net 3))
 (via (at 68.75 45.335) (size 0.6) (drill 0.4) (layers F.Cu B.Cu) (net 3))
 (segment (start 78 52.085) (end 78 52.835) (width 0.6) (layer F.Cu) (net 4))
 (segment (start 75 52.835) (end 75.75 52.835) (width 0.6) (layer B.Cu) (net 4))
 (via (at 75.75 52.835) (size 0.6) (drill 0.4) (layers F.Cu B.Cu) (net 4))
 (segment (start 72 52.835) (end 71.25 52.835) (width 0.6) (layer F.Cu) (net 4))
 (via (at 71.25 52.835) (size 0.6) (drill 0.4) (layers F.Cu B.Cu) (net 4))
 (segment (start 72.75 52.835) (end 72 52.835) (width 0.6) (layer B.Cu) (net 4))
 (via (at 72 52.835) (size 0.6) (drill 0.4) (layers F.Cu B.Cu) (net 4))
 (segment (start 73.5 52.835) (end 72.75 52.835) (width 0.6) (layer F.Cu) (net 4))
 (via (at 72.75 52.835) (size 0.6) (drill 0.4) (layers F.Cu B.Cu) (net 4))
 (segment (start 74.25 52.835) (end 73.5 52.835) (width 0.6) (layer B.Cu) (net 4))
 (via (at 73.5 52.835) (size 0.6) (drill 0.4) (layers F.Cu B.Cu) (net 4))
 (segment (start 75 52.835) (end 74.25 52.835) (width 0.6) (layer F.Cu) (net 4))
 (via (at 74.25 52.835) (size 0.6) (drill 0.4) (layers F.Cu B.Cu) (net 4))
 (via (at 75 52.835) (size 0.6) (drill 0.4) (layers F.Cu B.Cu) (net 4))
 (segment (start 76.5 52.835) (end 75.75 52.835) (width 0.6) (layer B.Cu) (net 4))
 (segment (start 77.25 52.835) (end 76.5 52.835) (width 0.6) (layer F.Cu) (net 4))
 (via (at 76.5 52.835) (size 0.6) (drill 0.4) (layers F.Cu B.Cu) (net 4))
 (segment (start 78 52.835) (end 77.25 52.835) (width 0.6) (layer B.Cu) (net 4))
 (via (at 77.25 52.835) (size 0.6) (drill 0.4) (layers F.Cu B.Cu) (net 4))
 (via (at 78 52.835) (size 0.6) (drill 0.4) (layers F.Cu B.Cu) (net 4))
 (segment (start 77.25 52.085) (end 78 52.085) (width 0.6) (layer B.Cu) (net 4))
 (via (at 78 52.085) (size 0.6) (drill 0.4) (layers F.Cu B.Cu) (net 4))
 (segment (start 76.5 52.085) (end 77.25 52.085) (width 0.6) (layer F.Cu) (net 4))
 (via (at 77.25 52.085) (size 0.6) (drill 0.4) (layers F.Cu B.Cu) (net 4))
 (segment (start 75.75 52.085) (end 76.5 52.085) (width 0.6) (layer B.Cu) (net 4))
 (via (at 76.5 52.085) (size 0.6) (drill 0.4) (layers F.Cu B.Cu) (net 4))
 (segment (start 75 52.085) (end 75.75 52.085) (width 0.6) (layer F.Cu) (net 4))
 (via (at 75.75 52.085) (size 0.6) (drill 0.4) (layers F.Cu B.Cu) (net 4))
 (segment (start 74.25 52.085) (end 75 52.085) (width 0.6) (layer B.Cu) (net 4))
 (via (at 75 52.085) (size 0.6) (drill 0.4) (layers F.Cu B.Cu) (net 4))
 (segment (start 73.5 52.085) (end 74.25 52.085) (width 0.6) (layer F.Cu) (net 4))
 (via (at 74.25 52.085) (size 0.6) (drill 0.4) (layers F.Cu B.Cu) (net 4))
 (segment (start 72.75 52.085) (end 73.5 52.085) (width 0.6) (layer B.Cu) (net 4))
 (via (at 73.5 52.085) (size 0.6) (drill 0.4) (layers F.Cu B.Cu) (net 4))
 (segment (start 72 52.085) (end 72.75 52.085) (width 0.6) (layer F.Cu) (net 4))
 (via (at 72.75 52.085) (size 0.6) (drill 0.4) (layers F.Cu B.Cu) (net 4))
 (segment (start 71.25 52.085) (end 72 52.085) (width 0.6) (layer B.Cu) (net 4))
 (via (at 72 52.085) (size 0.6) (drill 0.4) (layers F.Cu B.Cu) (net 4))
 (segment (start 70.35 52.085) (end 71.25 52.085) (width 0.6) (layer F.Cu) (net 4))
 (via (at 71.25 52.085) (size 0.6) (drill 0.4) (layers F.Cu B.Cu) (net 4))
 (segment (start 68.6 53.835) (end 69.85 52.585) (width 0.6) (layer F.Cu) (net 4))
 (segment (start 69.85 52.585) (end 70.35 52.085) (width 0.6) (layer F.Cu) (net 4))
 (segment (start 70.35 52.085) (end 72.45 49.985) (width 0.6) (layer F.Cu) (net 4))
 (segment (start 72.45 46.685) (end 71.074998 46.685) (width 0.6) (layer F.Cu) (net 4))
 (segment (start 71.074998 46.685) (end 70.175 47.584998) (width 0.6) (layer F.Cu) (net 4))
 (segment (start 70.175 47.584998) (end 70.175 48.635) (width 0.6) (layer F.Cu) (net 4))
 (segment (start 70.175 48.635) (end 70.525 48.985) (width 0.6) (layer F.Cu) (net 4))
 (segment (start 70.525 48.985) (end 72.45 48.985) (width 0.6) (layer F.Cu) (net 4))
 (segment (start 72.275 45.185) (end 76.675 45.185) (width 0.6) (layer F.Cu) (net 4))
 (segment (start 72.275 50.485) (end 76.675 50.485) (width 0.6) (layer F.Cu) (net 4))
 (via (at 71 44.335) (size 0.6) (drill 0.4) (layers F.Cu B.Cu) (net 4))
 (via (at 71.75 44.335) (size 0.6) (drill 0.4) (layers F.Cu B.Cu) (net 4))
 (via (at 73.25 44.335) (size 0.6) (drill 0.4) (layers F.Cu B.Cu) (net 4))
 (via (at 72.5 44.335) (size 0.6) (drill 0.4) (layers F.Cu B.Cu) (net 4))
 (via (at 78 51.085) (size 0.6) (drill 0.4) (layers F.Cu B.Cu) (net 4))
 (via (at 77.25 51.085) (size 0.6) (drill 0.4) (layers F.Cu B.Cu) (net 4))
 (via (at 76.5 51.085) (size 0.6) (drill 0.4) (layers F.Cu B.Cu) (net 4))
 (via (at 75.75 51.085) (size 0.6) (drill 0.4) (layers F.Cu B.Cu) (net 4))
 (via (at 73.5 51.085) (size 0.6) (drill 0.4) (layers F.Cu B.Cu) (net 4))
 (via (at 72.75 51.085) (size 0.6) (drill 0.4) (layers F.Cu B.Cu) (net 4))
 (via (at 72 51.085) (size 0.6) (drill 0.4) (layers F.Cu B.Cu) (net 4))
 (via (at 71.25 51.085) (size 0.6) (drill 0.4) (layers F.Cu B.Cu) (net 4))
 (via (at 77.75 44.335) (size 0.6) (drill 0.4) (layers F.Cu B.Cu) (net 4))
 (via (at 77 44.335) (size 0.6) (drill 0.4) (layers F.Cu B.Cu) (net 4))
 (via (at 76.25 44.335) (size 0.6) (drill 0.4) (layers F.Cu B.Cu) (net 4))
 (via (at 75.5 44.335) (size 0.6) (drill 0.4) (layers F.Cu B.Cu) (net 4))
 (segment (start 55.96 51.835) (end 55.96 53.27184) (width 0.6) (layer F.Cu) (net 4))
 (segment (start 55.96 53.27184) (end 56.52316 53.835) (width 0.6) (layer F.Cu) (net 4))
 (segment (start 56.52316 53.835) (end 68.6 53.835) (width 0.6) (layer F.Cu) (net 4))
 (segment (start 72.45 49.985) (end 72.45 48.985) (width 0.6) (layer F.Cu) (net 4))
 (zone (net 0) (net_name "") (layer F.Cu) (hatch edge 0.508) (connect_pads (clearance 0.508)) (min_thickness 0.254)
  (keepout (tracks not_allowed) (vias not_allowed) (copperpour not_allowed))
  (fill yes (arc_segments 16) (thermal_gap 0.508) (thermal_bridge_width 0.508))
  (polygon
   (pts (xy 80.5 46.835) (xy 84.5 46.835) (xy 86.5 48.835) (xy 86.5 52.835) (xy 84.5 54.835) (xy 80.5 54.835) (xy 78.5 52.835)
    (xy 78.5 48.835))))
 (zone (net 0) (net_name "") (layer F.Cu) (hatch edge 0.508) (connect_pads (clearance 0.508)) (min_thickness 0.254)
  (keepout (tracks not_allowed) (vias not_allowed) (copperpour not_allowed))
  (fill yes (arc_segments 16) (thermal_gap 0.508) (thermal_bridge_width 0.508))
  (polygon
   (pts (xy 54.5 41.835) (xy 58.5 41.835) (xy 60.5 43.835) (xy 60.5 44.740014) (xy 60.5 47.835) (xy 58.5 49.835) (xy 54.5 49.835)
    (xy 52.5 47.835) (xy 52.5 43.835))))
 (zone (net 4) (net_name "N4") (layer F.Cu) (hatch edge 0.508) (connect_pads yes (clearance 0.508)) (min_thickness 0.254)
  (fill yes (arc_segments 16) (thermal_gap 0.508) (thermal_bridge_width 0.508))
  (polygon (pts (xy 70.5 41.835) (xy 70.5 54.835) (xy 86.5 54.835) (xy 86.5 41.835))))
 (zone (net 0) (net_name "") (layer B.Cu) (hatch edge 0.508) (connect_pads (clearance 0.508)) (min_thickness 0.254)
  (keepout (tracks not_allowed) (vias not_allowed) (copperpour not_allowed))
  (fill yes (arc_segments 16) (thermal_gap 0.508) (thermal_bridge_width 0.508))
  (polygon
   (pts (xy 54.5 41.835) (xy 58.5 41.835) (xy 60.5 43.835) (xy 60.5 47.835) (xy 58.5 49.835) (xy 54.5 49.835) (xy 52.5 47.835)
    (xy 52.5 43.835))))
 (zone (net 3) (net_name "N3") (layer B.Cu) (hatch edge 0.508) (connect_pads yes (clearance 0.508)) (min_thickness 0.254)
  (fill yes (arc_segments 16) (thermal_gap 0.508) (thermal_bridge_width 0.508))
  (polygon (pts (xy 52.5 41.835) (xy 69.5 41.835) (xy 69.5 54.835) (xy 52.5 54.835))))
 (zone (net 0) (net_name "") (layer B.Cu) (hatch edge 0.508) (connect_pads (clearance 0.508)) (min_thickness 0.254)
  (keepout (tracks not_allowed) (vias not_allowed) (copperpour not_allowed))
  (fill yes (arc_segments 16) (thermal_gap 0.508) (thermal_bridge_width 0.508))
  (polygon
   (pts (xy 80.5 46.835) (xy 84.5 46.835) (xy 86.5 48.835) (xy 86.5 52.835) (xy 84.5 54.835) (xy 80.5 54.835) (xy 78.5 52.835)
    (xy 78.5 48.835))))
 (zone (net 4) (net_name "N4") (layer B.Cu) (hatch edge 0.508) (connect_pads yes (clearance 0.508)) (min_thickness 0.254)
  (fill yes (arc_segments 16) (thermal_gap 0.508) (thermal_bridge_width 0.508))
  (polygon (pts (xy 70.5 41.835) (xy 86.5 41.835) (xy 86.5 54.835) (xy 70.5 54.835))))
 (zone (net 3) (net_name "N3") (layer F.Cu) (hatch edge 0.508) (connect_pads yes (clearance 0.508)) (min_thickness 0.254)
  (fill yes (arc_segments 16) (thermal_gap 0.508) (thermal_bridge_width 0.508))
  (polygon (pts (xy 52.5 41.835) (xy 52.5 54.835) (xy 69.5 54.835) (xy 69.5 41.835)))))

